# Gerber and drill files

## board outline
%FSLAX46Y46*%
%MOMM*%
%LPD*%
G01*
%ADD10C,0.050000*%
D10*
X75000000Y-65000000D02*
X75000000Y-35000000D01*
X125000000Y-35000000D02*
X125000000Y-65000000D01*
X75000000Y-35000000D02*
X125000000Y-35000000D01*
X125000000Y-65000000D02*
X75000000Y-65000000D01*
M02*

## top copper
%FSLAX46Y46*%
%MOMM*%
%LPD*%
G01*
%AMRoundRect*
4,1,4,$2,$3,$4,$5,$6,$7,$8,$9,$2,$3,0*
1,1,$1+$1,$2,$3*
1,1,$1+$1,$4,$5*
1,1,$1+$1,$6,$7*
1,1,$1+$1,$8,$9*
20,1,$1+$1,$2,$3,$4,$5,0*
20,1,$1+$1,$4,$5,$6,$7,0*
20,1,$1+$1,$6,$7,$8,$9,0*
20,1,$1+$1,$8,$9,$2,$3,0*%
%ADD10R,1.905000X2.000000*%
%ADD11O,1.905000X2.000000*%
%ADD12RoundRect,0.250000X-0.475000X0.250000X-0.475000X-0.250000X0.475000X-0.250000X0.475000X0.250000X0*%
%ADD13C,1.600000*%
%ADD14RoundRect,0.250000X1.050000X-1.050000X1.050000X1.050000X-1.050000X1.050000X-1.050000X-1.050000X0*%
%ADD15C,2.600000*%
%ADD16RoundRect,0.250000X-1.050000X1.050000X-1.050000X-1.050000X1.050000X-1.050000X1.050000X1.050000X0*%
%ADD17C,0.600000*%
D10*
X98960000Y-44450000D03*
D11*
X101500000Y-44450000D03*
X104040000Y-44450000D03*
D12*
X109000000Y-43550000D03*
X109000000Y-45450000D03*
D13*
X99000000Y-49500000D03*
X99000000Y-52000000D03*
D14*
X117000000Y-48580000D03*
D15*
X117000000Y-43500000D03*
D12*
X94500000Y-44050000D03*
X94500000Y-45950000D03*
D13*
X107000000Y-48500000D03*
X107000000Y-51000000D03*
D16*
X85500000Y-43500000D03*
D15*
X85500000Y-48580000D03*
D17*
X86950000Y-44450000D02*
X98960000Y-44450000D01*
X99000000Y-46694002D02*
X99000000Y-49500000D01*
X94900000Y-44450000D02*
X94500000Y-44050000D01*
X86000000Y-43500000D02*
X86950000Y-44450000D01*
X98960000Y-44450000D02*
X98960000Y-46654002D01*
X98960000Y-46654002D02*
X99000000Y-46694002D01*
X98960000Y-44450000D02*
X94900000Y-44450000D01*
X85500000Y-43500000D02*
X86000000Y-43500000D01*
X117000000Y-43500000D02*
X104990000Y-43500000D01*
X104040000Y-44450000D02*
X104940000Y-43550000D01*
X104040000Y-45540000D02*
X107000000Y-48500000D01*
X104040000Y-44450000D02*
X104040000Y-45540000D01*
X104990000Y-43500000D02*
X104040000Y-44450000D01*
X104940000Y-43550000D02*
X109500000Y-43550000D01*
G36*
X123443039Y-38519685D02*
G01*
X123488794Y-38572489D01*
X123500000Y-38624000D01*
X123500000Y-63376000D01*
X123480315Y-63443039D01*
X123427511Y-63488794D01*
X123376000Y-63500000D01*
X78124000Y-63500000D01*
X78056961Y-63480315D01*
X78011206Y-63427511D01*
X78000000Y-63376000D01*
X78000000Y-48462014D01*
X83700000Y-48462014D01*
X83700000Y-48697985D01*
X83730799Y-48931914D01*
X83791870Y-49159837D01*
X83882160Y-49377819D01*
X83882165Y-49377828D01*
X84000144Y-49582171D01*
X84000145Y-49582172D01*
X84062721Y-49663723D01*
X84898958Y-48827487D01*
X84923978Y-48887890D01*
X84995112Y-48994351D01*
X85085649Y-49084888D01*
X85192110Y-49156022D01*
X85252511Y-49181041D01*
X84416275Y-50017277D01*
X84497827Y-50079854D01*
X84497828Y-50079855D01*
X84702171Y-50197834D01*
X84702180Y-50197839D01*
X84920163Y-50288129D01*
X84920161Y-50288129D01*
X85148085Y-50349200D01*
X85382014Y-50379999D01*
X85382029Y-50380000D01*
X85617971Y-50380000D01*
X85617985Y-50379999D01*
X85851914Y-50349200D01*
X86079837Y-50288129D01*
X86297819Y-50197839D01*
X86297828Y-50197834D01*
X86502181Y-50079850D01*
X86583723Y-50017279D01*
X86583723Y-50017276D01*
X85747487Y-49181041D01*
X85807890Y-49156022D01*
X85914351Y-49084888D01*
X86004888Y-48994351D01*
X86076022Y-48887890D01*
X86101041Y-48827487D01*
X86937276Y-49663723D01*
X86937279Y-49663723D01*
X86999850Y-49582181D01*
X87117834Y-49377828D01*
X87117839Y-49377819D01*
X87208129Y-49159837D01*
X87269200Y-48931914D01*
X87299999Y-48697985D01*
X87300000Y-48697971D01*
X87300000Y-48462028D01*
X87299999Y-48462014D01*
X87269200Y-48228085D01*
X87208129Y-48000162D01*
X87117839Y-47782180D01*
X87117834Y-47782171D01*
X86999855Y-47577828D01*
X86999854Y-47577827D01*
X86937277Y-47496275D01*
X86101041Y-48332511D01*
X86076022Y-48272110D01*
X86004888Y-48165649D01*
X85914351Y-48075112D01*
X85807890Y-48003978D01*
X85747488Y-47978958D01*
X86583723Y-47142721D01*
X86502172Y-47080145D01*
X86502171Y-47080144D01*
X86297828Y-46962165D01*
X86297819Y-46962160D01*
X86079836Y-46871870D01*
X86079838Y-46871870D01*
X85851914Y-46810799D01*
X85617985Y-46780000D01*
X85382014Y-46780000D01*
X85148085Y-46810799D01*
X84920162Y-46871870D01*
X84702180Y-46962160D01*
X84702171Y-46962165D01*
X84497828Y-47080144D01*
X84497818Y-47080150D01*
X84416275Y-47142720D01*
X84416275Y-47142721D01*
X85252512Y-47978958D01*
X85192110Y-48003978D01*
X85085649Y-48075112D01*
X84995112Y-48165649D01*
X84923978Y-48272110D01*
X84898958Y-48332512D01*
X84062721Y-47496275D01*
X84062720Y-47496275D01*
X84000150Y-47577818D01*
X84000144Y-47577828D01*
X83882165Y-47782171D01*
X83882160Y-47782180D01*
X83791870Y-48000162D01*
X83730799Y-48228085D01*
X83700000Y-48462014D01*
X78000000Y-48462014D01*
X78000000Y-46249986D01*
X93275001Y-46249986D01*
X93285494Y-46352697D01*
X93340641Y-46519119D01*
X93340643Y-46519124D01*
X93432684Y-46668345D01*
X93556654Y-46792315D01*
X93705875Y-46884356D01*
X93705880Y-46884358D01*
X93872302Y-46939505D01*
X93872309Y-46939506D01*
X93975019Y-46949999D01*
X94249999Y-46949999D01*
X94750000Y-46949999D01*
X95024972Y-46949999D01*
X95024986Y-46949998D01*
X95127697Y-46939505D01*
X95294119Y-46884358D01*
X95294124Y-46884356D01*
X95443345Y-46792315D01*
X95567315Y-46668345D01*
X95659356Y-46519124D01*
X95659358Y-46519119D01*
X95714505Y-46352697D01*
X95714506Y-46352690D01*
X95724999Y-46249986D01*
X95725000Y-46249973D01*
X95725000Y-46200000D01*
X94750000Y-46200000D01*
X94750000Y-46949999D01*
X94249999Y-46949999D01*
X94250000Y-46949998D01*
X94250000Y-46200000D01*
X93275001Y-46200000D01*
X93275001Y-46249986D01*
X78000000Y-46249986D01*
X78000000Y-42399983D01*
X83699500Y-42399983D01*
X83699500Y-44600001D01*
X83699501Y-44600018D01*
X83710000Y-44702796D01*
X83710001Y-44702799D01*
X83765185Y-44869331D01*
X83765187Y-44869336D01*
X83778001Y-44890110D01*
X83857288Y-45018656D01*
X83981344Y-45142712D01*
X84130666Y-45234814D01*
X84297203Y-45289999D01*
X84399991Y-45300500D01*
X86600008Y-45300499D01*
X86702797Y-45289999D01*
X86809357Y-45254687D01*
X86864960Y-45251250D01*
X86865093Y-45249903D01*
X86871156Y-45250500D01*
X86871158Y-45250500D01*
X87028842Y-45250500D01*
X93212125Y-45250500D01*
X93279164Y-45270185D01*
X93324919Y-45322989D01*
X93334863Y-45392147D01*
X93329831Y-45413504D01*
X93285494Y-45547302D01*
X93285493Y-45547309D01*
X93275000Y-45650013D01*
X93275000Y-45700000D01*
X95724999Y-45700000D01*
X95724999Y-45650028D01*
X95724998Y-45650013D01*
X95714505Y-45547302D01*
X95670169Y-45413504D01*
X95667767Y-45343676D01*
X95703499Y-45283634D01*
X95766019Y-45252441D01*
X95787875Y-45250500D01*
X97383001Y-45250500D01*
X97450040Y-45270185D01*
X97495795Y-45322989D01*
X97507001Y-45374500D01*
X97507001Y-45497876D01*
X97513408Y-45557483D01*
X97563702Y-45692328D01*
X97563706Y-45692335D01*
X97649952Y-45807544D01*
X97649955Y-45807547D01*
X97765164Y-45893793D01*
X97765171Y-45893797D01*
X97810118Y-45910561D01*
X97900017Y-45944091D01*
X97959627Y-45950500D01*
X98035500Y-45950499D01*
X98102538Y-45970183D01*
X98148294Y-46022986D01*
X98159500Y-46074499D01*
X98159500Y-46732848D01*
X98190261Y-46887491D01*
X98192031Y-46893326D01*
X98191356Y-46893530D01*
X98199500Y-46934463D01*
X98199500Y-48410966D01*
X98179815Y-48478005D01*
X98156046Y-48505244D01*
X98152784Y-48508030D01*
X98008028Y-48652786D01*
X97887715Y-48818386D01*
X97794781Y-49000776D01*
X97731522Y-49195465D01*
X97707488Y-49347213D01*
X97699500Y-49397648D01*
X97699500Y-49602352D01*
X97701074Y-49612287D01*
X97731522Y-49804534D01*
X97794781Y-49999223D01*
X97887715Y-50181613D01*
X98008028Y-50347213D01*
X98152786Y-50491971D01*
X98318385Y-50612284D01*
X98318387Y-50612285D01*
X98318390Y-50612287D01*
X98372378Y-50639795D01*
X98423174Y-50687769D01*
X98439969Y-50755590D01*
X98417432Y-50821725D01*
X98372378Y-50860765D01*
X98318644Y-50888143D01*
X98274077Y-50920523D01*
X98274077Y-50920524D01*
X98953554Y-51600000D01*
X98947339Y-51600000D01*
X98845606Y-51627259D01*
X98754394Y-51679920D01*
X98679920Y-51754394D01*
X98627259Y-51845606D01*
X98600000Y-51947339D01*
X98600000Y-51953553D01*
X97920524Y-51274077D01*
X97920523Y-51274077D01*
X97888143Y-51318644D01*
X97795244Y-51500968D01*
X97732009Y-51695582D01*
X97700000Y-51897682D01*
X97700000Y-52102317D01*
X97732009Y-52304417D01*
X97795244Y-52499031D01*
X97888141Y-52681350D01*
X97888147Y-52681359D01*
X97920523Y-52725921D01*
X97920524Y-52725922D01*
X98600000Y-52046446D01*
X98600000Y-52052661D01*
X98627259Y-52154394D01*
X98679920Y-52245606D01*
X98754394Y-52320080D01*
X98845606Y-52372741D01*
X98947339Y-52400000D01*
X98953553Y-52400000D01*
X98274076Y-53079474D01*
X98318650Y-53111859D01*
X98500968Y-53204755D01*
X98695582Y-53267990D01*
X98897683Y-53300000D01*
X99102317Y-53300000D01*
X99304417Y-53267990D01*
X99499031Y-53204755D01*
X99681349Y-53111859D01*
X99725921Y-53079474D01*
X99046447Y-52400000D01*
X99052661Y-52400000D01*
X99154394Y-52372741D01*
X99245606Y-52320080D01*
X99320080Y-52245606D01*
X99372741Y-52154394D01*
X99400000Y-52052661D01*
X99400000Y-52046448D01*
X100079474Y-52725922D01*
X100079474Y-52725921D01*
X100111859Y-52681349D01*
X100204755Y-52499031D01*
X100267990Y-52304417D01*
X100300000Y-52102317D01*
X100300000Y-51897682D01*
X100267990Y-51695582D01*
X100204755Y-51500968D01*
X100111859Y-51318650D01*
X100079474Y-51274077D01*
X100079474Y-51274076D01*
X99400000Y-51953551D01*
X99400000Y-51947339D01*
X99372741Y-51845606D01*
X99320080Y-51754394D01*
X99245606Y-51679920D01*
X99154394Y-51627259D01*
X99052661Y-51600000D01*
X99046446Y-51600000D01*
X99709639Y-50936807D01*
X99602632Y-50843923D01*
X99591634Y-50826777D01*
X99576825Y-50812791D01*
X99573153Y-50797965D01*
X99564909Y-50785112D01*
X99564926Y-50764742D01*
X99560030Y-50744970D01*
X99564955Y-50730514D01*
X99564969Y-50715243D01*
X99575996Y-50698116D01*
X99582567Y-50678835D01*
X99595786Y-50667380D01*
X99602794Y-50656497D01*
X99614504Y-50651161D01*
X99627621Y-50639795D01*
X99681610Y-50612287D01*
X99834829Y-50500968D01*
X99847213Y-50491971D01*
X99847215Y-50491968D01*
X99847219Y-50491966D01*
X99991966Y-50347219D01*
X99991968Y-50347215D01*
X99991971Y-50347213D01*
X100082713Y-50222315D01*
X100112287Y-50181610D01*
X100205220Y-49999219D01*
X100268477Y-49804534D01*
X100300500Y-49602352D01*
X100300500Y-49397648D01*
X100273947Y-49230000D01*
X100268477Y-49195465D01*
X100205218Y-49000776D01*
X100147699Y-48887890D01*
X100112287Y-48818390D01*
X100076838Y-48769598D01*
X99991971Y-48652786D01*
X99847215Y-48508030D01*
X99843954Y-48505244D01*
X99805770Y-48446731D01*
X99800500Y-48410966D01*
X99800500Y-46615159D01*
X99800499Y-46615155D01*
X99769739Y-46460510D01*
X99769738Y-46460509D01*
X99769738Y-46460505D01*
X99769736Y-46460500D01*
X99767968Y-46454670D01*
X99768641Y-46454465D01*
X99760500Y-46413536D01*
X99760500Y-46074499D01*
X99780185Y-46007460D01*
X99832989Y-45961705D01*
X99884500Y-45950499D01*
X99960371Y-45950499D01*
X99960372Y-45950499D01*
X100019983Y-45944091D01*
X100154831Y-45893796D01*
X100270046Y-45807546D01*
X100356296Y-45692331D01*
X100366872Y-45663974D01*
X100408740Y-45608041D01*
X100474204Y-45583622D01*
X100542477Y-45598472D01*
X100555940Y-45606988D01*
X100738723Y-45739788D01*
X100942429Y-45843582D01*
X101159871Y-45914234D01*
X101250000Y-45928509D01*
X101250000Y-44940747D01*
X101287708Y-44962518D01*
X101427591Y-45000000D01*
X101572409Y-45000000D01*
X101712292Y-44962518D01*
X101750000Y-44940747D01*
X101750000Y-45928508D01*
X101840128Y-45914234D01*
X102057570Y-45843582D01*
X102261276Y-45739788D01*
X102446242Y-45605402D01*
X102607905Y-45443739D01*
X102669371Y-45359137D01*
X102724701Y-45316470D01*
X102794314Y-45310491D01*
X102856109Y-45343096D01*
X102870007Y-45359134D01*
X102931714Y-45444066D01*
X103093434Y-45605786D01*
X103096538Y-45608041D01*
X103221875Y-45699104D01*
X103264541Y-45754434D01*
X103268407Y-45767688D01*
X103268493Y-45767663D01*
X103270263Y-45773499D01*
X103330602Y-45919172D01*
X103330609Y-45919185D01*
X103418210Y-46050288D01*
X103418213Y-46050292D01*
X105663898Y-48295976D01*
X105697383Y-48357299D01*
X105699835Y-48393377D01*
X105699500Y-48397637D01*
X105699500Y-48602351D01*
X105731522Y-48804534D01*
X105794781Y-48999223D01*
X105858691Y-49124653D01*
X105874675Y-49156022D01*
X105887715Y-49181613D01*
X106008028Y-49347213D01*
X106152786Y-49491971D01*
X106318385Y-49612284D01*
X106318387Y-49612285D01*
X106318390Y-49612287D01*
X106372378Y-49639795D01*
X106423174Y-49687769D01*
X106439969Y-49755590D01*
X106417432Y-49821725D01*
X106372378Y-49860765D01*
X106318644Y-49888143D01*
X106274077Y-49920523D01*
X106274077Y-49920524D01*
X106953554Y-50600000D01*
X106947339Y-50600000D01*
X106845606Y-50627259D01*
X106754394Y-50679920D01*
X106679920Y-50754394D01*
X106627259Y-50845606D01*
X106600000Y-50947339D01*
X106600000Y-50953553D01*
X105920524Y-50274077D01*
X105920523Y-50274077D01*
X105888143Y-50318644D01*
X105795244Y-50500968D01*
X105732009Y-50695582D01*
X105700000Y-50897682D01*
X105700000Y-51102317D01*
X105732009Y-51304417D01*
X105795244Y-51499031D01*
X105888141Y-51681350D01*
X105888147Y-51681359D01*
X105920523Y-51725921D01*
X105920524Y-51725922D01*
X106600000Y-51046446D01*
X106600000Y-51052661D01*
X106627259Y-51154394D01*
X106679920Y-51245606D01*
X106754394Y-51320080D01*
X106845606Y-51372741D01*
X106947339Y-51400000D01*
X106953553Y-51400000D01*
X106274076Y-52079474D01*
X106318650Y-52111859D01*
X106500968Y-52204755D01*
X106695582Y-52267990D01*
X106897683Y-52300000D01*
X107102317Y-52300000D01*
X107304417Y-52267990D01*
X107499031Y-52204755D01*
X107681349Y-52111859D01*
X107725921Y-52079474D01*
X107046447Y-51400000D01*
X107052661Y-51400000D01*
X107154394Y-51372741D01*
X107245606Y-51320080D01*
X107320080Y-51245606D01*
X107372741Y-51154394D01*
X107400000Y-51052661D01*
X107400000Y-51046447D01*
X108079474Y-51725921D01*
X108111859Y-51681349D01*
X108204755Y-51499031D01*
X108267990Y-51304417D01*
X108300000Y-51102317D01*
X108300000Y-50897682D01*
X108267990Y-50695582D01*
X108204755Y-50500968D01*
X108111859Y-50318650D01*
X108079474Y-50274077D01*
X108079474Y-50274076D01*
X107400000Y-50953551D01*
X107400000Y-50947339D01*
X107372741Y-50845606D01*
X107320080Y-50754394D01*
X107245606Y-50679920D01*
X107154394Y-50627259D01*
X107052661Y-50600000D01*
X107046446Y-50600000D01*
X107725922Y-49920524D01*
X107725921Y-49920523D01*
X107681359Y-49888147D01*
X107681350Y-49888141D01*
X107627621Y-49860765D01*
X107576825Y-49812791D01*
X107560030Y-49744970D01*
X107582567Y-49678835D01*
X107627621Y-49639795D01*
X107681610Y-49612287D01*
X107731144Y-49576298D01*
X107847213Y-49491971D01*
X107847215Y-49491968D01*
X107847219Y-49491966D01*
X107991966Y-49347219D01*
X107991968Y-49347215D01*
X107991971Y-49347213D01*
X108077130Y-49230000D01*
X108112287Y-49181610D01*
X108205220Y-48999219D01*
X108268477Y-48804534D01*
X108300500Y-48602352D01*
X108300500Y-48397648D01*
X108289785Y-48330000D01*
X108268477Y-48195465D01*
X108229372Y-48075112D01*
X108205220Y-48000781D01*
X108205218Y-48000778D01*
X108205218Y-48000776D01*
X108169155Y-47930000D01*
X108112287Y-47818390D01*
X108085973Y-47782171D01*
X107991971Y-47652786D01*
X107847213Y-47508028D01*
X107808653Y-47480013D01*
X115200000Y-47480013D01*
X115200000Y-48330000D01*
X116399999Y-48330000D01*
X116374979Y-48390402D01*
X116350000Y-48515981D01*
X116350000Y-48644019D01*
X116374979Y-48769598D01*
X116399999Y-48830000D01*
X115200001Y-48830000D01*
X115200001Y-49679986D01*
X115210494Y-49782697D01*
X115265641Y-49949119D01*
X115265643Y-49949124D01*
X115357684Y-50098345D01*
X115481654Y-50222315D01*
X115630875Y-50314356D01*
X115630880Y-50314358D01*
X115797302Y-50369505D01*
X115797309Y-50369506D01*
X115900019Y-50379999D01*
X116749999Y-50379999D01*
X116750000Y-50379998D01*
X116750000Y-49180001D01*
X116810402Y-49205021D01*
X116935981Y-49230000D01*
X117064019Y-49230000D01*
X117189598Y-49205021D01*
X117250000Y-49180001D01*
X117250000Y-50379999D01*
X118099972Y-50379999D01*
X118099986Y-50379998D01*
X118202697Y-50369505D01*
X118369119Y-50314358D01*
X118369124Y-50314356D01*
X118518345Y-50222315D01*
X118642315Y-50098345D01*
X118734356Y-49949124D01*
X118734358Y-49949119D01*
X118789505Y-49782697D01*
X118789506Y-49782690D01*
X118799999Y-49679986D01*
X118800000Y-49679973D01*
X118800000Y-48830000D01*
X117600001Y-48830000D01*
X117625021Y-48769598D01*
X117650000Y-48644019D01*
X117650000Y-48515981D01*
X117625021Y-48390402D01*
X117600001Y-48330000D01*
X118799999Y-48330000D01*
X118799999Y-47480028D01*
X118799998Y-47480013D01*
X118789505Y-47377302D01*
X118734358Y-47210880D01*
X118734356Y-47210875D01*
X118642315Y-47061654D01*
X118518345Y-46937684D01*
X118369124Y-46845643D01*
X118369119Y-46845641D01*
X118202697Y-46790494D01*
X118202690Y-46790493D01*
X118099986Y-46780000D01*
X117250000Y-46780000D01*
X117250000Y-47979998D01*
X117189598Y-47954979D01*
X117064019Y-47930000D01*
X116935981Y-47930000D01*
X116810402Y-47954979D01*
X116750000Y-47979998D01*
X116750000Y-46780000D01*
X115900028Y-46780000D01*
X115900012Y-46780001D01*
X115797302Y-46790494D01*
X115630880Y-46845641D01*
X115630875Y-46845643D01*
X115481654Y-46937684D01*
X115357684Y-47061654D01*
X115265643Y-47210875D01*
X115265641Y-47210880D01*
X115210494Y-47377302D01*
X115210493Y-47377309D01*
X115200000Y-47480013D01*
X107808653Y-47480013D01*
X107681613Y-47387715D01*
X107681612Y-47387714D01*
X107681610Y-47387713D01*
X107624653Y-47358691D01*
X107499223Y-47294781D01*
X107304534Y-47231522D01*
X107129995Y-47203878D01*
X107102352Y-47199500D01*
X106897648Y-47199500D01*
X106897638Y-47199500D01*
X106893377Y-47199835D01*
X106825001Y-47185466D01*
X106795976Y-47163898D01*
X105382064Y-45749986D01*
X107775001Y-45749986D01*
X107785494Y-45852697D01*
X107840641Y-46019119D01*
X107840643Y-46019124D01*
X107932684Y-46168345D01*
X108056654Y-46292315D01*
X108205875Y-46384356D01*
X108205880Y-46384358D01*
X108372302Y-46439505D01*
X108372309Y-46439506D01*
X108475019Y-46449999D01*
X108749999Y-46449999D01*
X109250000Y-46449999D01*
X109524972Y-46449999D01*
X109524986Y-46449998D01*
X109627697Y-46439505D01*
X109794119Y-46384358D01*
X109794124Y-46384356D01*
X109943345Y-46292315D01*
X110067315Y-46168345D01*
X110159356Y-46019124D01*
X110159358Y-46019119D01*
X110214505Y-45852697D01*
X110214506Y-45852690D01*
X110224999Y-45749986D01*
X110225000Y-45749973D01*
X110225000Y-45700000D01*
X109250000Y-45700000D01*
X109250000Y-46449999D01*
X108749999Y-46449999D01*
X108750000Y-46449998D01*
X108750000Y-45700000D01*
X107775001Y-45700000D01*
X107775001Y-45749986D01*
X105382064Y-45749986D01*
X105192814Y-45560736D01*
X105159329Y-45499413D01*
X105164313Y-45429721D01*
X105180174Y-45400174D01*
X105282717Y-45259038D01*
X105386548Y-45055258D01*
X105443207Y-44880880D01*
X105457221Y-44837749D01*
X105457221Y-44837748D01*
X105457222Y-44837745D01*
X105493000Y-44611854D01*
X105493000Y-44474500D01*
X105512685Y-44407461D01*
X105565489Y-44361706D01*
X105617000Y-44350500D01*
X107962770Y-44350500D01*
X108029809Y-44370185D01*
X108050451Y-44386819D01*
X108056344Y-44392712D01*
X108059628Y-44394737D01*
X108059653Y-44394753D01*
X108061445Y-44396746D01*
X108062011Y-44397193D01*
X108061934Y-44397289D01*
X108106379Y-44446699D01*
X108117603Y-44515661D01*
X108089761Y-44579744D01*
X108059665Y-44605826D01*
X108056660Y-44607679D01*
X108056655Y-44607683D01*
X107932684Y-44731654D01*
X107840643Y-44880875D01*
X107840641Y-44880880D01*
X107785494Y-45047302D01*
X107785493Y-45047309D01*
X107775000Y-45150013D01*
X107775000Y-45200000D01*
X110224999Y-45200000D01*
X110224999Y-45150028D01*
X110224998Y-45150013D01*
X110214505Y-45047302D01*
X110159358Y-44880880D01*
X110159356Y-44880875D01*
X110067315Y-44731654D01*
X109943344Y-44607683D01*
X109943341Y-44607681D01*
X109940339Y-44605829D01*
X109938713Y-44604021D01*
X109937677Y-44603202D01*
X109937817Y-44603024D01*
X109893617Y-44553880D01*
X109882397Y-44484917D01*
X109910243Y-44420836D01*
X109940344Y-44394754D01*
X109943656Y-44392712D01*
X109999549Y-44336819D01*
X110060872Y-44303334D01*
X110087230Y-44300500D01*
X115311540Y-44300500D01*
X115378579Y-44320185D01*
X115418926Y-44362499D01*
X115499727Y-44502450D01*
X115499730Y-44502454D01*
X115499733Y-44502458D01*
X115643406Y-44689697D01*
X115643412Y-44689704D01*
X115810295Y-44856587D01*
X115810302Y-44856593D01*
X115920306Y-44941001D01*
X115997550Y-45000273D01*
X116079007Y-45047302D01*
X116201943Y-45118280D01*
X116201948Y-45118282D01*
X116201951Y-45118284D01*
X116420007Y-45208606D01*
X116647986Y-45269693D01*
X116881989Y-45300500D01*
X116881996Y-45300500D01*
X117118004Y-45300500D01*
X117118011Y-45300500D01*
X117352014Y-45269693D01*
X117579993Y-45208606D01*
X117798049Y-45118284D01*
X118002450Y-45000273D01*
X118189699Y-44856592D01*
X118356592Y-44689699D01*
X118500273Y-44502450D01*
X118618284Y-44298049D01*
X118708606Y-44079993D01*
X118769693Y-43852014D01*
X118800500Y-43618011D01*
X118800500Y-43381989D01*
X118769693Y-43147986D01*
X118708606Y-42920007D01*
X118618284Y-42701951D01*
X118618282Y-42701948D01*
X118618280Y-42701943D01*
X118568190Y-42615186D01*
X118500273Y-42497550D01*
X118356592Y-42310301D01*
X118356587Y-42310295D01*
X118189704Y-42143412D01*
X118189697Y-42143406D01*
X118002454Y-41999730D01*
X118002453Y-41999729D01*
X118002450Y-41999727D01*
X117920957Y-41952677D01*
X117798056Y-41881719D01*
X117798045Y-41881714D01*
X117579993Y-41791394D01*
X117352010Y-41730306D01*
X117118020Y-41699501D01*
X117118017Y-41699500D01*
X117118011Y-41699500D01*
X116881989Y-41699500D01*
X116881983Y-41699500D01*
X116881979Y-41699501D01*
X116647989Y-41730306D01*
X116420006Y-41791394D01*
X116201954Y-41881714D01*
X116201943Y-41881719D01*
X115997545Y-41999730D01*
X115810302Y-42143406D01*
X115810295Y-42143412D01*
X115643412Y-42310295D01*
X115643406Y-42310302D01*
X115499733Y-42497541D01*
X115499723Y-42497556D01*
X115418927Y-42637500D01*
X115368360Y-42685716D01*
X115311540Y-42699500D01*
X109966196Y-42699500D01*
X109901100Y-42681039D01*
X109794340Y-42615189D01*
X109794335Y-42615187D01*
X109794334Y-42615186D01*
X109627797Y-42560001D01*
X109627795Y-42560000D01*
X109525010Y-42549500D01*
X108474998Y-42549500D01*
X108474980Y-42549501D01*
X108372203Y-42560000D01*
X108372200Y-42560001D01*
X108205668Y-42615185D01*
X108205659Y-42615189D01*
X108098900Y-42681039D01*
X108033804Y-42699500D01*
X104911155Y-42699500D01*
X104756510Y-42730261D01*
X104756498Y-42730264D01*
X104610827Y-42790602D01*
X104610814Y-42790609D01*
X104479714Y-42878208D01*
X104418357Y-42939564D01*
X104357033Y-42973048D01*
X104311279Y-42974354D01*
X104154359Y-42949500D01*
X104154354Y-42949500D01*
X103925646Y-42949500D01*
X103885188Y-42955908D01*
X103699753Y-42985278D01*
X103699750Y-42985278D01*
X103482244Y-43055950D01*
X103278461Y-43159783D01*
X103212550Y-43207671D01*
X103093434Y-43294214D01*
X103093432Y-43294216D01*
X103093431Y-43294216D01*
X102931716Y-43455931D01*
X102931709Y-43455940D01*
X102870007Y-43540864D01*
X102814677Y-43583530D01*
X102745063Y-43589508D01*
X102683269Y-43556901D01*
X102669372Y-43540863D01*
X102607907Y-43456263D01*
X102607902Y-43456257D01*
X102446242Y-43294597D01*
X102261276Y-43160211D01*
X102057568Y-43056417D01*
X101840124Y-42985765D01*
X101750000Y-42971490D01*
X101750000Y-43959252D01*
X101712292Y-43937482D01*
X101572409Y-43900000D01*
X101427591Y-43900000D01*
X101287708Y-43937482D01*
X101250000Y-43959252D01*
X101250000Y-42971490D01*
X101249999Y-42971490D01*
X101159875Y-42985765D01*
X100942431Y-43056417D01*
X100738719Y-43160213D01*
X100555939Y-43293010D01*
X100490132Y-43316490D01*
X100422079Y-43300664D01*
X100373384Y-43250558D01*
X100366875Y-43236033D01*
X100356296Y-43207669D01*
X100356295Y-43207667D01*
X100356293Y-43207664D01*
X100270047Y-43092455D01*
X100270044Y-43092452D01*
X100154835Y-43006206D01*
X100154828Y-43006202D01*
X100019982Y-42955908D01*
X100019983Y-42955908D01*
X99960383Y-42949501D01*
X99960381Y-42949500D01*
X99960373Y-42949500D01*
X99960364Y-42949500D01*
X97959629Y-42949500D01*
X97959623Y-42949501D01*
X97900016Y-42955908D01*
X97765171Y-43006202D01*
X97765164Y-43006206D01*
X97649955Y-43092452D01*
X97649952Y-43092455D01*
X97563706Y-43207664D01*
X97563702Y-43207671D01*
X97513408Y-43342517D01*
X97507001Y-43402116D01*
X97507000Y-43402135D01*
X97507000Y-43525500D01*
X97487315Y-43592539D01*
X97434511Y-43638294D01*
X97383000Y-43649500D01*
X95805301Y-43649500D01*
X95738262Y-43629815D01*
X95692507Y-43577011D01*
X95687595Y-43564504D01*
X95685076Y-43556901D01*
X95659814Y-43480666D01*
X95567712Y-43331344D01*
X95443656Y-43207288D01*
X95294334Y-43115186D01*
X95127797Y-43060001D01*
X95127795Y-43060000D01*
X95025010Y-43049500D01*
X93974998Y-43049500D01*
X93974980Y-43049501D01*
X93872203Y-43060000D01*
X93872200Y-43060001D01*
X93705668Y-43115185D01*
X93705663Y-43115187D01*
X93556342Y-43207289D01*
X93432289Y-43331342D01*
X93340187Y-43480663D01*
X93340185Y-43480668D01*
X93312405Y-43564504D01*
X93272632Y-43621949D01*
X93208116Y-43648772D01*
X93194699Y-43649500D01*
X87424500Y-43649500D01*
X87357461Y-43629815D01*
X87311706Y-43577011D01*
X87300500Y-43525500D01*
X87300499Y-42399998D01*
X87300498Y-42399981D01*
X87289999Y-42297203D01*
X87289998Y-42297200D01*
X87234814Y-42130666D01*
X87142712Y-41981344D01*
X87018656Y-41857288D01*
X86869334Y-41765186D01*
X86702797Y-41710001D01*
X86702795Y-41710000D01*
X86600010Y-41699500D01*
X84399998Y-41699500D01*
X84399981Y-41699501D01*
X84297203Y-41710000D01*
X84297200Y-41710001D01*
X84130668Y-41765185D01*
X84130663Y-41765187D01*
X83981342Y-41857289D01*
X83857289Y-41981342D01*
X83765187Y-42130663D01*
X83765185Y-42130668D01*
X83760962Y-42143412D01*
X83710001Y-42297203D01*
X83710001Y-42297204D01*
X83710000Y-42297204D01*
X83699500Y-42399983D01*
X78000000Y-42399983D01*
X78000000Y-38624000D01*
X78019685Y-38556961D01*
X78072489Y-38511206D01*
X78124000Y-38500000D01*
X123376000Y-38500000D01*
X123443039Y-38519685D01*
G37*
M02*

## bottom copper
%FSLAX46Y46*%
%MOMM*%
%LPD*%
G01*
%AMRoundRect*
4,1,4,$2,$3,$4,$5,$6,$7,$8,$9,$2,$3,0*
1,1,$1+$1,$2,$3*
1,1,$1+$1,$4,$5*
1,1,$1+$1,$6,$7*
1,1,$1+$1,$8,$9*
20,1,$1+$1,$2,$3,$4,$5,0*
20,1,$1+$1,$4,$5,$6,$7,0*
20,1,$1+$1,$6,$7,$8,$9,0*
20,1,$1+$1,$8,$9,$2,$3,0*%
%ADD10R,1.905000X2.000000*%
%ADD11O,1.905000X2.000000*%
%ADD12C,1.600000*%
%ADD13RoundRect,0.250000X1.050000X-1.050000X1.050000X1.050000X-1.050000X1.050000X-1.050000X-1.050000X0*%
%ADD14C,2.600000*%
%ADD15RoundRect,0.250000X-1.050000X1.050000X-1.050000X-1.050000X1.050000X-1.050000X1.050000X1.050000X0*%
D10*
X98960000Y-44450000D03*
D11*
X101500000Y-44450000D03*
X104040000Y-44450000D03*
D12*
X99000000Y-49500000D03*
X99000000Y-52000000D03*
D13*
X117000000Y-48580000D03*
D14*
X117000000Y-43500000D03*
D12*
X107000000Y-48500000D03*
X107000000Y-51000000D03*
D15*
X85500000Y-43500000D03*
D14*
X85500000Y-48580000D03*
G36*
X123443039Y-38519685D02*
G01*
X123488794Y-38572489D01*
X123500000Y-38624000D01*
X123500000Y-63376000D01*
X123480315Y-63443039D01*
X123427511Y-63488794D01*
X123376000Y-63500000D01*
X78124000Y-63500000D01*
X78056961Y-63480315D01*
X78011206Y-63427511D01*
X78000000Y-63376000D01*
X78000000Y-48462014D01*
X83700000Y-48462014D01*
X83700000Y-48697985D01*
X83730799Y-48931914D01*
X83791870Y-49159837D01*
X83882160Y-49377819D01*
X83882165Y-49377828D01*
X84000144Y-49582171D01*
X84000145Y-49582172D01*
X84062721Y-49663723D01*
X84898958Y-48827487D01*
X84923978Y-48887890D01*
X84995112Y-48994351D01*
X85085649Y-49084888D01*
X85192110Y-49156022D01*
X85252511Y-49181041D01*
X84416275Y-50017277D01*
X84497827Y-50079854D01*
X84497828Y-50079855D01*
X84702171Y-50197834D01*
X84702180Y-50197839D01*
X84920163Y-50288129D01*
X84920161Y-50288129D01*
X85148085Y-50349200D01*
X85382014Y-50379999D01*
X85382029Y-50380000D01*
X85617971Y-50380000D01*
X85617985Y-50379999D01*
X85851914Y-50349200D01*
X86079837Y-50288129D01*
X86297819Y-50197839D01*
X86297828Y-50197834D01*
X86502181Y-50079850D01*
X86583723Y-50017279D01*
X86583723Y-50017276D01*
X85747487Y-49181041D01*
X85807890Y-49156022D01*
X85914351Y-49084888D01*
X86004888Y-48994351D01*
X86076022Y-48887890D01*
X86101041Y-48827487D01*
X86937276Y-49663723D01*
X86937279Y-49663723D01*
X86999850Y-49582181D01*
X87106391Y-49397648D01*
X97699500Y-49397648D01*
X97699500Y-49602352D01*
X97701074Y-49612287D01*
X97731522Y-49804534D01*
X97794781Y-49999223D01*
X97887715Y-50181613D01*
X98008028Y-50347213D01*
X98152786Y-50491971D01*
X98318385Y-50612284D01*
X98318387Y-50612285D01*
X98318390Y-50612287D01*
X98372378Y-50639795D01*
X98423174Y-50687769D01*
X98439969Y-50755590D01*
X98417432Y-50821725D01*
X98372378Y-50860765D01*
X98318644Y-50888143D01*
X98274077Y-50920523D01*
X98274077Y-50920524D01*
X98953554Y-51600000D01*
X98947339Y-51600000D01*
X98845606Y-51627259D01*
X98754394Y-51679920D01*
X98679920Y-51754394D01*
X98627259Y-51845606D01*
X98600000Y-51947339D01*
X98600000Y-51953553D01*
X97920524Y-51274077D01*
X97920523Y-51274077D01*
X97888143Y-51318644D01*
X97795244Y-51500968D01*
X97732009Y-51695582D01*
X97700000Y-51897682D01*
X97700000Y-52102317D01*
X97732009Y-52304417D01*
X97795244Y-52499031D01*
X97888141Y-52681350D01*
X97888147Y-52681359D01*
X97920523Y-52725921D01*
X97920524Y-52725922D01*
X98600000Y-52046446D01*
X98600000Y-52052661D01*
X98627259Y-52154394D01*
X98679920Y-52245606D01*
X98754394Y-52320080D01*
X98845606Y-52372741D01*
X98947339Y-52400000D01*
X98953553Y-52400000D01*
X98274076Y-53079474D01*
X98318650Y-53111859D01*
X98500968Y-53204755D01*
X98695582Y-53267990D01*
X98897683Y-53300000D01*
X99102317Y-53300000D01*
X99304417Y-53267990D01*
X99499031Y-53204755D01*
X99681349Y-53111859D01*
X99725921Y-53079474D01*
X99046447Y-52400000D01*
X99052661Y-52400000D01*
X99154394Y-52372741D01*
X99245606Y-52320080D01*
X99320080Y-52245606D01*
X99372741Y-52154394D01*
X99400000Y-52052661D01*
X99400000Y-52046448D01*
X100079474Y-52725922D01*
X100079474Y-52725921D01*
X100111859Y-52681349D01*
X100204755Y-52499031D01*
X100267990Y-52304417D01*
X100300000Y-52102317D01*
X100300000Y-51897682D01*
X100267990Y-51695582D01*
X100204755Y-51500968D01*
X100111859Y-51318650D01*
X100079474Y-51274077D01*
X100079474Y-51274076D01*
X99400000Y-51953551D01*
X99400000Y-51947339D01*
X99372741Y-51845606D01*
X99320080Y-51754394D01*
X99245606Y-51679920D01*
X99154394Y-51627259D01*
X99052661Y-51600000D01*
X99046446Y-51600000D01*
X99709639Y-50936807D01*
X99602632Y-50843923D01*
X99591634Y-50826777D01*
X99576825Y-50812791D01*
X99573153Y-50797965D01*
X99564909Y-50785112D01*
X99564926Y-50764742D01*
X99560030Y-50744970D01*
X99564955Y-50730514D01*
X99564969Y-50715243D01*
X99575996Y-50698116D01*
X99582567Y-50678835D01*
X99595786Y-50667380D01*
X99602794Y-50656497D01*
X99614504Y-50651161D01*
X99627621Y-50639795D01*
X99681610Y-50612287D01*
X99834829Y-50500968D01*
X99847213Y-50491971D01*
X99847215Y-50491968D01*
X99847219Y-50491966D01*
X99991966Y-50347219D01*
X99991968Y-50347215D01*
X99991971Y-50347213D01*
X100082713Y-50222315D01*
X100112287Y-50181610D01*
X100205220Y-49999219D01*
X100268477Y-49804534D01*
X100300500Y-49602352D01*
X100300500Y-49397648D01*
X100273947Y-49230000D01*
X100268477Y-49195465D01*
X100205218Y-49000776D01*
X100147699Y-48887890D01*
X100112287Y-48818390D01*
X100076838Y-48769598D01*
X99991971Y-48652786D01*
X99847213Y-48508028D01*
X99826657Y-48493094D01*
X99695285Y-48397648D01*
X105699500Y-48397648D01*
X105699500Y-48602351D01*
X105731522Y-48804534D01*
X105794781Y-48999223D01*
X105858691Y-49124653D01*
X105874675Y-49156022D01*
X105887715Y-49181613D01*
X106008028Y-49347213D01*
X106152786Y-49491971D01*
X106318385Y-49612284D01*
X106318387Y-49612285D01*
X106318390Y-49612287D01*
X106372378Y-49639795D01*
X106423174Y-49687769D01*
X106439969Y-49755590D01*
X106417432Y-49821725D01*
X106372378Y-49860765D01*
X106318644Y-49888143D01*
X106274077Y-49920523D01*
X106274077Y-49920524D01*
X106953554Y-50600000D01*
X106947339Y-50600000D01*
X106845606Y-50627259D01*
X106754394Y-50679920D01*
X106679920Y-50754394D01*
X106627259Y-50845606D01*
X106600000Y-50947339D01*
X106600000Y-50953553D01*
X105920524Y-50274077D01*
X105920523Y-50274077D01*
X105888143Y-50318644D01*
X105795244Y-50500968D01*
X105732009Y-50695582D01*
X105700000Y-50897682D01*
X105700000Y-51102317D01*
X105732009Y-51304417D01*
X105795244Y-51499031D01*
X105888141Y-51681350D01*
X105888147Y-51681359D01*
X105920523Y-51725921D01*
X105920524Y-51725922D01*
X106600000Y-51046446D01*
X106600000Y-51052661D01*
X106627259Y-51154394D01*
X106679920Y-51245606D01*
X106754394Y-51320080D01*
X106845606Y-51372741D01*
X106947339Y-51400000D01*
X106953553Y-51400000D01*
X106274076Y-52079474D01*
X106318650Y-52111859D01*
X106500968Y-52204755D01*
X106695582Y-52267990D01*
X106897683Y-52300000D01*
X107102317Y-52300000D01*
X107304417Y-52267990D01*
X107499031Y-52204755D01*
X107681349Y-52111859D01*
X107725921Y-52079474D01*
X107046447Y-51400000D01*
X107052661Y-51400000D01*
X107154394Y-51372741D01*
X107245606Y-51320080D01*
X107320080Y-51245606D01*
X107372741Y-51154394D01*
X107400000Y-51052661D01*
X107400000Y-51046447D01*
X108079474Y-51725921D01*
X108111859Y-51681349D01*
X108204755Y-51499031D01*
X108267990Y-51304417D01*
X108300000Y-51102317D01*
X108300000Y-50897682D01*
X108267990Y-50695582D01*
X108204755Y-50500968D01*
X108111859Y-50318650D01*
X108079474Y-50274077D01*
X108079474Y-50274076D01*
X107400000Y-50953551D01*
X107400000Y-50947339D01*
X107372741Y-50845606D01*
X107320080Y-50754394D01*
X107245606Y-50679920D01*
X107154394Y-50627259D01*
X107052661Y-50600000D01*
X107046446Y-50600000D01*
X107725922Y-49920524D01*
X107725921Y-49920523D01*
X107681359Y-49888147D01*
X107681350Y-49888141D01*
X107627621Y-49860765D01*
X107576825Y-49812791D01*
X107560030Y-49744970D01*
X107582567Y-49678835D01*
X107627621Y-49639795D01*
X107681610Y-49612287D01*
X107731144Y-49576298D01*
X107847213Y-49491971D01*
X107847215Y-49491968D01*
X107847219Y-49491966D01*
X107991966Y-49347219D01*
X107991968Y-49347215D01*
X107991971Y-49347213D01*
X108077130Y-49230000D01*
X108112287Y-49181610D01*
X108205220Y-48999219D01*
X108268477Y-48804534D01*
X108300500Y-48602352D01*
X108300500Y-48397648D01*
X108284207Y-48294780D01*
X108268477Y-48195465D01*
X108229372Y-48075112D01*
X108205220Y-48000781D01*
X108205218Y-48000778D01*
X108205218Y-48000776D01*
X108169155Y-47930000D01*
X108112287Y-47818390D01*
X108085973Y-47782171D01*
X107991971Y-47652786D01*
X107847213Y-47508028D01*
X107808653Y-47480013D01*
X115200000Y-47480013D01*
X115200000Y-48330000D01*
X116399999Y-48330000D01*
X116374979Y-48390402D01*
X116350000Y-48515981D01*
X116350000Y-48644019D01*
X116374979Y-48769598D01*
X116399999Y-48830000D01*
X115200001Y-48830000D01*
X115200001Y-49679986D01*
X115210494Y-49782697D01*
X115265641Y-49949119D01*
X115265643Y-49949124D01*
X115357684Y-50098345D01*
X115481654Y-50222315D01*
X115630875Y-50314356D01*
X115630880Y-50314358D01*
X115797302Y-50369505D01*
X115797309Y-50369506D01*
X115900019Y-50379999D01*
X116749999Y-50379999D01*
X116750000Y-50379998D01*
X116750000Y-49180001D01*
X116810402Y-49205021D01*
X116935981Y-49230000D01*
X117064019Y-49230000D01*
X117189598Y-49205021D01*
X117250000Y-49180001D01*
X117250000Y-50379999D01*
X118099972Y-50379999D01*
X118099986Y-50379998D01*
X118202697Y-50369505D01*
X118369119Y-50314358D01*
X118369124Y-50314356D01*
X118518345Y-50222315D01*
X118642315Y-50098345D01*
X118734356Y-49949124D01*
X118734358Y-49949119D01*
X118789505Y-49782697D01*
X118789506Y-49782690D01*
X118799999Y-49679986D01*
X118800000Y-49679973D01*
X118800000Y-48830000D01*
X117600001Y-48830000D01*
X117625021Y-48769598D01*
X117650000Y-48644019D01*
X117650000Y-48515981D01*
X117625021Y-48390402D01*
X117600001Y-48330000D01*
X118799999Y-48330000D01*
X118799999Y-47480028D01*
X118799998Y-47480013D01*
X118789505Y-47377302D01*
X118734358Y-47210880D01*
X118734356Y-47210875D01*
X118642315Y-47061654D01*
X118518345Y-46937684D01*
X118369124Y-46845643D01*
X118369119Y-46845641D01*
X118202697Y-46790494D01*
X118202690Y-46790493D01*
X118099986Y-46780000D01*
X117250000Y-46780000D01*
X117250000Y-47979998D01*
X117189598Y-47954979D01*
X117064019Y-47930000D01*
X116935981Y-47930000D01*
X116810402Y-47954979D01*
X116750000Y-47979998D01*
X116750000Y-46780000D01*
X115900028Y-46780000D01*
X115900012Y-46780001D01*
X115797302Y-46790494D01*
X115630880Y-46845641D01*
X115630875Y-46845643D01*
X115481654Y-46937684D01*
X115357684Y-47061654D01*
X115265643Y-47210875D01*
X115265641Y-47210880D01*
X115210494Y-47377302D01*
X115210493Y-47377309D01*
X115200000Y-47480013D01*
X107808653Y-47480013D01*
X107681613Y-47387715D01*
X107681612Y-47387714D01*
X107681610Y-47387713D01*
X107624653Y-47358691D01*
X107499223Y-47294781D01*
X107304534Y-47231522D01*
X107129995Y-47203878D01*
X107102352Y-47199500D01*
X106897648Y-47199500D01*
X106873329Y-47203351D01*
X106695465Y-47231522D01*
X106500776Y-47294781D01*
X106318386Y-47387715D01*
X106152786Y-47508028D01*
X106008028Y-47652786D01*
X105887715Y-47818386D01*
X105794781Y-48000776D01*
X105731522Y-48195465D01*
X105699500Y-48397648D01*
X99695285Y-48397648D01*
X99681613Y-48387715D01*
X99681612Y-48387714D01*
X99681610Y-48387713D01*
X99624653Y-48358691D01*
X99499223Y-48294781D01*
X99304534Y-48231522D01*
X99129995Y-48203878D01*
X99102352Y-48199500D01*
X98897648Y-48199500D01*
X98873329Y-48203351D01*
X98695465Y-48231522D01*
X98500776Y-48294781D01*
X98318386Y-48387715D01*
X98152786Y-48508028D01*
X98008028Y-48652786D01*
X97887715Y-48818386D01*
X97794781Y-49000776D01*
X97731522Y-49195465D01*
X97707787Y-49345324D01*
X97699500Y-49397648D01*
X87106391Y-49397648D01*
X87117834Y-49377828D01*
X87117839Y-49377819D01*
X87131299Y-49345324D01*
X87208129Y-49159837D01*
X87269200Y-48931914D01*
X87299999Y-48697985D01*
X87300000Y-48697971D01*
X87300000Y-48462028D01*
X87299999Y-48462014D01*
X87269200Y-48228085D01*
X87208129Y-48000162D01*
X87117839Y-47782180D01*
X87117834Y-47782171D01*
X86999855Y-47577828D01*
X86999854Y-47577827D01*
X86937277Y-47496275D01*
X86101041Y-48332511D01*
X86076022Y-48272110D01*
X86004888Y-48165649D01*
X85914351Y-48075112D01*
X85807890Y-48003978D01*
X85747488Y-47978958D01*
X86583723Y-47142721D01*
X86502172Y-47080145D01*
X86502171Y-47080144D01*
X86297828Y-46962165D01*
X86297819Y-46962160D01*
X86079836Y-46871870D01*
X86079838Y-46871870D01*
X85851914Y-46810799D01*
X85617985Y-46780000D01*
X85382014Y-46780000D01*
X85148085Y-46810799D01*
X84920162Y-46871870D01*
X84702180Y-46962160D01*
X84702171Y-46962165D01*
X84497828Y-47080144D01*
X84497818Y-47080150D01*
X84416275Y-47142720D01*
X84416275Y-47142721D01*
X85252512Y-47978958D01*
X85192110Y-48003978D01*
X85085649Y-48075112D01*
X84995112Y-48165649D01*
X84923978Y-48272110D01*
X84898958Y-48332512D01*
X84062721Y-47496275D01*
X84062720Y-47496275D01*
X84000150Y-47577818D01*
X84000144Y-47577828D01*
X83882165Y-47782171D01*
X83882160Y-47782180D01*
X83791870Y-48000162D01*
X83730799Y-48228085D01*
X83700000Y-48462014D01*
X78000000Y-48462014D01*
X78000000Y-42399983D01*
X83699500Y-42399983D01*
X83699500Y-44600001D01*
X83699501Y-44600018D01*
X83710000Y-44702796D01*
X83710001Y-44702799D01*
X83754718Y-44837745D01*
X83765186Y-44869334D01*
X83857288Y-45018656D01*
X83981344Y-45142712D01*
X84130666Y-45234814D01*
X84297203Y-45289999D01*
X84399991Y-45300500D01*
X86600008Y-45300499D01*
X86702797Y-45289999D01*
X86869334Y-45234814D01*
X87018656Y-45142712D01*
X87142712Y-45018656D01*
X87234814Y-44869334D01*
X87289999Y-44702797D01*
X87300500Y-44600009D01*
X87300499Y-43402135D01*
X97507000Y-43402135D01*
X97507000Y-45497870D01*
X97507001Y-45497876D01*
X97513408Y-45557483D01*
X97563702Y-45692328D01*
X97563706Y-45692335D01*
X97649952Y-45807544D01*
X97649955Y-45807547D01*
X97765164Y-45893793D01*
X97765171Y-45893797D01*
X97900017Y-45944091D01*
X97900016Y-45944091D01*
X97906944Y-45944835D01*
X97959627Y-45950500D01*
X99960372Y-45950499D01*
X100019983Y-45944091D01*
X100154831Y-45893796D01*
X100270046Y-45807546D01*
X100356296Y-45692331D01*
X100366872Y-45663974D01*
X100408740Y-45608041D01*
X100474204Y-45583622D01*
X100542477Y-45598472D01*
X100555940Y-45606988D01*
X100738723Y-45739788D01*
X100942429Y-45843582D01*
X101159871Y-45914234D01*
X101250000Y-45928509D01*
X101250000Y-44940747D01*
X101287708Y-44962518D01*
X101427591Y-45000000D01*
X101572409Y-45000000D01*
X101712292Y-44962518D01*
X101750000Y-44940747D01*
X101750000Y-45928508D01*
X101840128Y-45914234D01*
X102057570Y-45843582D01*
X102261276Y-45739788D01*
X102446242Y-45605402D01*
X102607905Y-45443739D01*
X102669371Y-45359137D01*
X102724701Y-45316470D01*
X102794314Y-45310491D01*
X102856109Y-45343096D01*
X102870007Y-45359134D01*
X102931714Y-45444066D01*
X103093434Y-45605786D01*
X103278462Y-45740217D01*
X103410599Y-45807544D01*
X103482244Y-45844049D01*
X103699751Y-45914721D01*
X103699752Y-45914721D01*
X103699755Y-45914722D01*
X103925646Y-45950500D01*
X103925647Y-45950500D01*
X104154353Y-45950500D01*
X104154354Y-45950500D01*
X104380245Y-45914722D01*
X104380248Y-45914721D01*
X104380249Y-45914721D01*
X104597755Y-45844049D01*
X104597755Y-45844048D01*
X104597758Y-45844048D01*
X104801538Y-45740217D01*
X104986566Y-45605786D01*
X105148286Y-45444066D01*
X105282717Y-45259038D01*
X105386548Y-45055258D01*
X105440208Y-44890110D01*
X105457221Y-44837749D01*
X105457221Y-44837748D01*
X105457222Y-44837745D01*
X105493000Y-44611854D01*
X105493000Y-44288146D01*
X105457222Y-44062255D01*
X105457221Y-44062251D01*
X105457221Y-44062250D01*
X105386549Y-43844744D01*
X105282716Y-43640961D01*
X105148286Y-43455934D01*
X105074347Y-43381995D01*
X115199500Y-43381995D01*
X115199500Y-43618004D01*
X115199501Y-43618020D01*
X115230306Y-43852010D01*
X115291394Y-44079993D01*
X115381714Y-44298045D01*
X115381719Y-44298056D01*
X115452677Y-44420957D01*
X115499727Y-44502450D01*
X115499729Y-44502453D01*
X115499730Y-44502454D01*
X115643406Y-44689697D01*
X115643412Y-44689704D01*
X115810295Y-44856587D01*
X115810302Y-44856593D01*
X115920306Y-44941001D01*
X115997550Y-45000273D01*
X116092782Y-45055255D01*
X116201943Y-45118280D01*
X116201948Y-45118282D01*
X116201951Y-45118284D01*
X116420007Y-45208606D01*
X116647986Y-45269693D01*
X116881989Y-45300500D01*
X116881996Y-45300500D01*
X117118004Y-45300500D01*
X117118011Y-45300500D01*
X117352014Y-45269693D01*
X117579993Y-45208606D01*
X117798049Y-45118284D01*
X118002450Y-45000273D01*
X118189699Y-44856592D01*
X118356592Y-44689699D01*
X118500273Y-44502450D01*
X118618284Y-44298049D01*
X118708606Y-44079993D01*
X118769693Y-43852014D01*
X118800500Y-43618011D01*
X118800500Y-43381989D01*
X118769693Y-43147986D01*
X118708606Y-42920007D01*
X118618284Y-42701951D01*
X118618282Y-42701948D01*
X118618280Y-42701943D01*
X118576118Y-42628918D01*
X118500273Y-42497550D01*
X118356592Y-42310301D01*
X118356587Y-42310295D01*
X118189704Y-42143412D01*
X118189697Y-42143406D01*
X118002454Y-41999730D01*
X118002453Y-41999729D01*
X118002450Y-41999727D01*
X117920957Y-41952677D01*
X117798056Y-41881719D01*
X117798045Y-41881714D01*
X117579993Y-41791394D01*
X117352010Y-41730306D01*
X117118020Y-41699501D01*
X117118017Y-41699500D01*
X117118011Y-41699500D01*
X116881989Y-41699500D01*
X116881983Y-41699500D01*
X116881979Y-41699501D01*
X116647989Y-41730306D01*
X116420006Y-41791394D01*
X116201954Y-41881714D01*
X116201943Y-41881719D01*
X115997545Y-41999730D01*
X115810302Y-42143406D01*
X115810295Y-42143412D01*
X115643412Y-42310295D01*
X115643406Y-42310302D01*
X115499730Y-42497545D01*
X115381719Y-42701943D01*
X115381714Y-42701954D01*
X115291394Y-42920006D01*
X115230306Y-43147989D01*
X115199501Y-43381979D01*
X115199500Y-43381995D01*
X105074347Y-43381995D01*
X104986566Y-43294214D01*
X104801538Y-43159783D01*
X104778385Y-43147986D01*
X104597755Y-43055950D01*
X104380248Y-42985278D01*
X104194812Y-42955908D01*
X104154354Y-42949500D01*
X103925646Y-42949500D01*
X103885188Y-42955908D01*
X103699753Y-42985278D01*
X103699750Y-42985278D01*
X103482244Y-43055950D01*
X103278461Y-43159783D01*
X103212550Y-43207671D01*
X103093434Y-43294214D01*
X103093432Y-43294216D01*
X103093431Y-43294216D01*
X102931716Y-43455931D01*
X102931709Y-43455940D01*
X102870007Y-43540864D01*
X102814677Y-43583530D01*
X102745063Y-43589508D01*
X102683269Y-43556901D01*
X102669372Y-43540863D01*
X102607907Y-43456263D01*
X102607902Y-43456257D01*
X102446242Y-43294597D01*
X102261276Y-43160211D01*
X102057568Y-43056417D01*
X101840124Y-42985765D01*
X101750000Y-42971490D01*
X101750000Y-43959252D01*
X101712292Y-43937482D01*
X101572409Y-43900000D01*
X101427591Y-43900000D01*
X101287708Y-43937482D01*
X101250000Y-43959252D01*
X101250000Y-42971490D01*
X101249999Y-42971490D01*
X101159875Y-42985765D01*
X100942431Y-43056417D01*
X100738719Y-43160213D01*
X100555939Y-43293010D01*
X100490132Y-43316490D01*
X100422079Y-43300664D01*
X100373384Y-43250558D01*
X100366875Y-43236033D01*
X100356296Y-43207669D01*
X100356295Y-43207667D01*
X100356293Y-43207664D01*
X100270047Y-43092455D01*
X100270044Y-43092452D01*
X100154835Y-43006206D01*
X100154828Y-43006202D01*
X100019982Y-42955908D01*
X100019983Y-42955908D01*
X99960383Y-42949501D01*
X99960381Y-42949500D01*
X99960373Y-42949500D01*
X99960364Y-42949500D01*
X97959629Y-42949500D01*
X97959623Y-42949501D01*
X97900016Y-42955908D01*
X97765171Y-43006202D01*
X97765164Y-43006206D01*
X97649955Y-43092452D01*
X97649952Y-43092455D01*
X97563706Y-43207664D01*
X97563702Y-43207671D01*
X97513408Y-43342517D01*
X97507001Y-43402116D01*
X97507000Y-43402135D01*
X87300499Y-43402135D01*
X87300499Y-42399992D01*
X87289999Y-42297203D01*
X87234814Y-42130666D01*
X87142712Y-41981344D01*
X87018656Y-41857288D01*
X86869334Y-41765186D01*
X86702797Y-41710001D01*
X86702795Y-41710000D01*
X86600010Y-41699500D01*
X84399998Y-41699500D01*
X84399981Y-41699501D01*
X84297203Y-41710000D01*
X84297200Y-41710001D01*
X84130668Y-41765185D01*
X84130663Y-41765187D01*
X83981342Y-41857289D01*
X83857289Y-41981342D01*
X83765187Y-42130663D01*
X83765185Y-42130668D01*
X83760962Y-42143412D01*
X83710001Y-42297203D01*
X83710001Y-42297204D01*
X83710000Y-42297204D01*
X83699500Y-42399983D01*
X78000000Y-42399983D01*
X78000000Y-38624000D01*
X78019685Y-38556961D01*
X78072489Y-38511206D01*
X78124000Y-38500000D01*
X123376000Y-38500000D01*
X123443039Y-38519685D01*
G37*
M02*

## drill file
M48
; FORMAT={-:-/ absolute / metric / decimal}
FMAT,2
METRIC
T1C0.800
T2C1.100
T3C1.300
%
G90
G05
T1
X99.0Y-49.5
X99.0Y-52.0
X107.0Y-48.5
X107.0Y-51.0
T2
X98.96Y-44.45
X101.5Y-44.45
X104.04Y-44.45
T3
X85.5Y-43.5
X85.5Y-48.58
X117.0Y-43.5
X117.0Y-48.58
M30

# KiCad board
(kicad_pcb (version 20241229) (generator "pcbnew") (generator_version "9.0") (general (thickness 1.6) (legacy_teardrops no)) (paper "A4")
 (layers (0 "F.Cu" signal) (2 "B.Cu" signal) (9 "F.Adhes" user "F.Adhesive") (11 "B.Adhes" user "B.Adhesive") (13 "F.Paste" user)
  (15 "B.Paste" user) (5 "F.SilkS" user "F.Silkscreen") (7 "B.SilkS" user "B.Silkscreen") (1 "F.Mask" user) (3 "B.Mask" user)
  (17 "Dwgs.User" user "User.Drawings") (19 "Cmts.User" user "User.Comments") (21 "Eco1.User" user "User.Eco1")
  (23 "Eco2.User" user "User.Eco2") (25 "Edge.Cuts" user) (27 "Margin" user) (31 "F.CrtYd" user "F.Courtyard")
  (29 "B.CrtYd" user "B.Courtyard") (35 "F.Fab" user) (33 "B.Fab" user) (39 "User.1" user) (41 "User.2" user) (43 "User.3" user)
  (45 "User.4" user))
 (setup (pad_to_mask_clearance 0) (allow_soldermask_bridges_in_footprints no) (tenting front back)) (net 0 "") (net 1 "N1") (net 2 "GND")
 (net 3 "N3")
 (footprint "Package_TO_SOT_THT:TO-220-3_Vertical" (layer "F.Cu") (at 98.96 44.45)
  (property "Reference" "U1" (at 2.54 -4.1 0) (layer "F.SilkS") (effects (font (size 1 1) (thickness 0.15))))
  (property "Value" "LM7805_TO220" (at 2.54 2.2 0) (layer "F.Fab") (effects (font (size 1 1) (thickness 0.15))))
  (pad "1" thru_hole rect (at 0 0) (size 1.905 2) (drill 1.1) (layers "*.Cu" "*.Mask") (remove_unused_layers no) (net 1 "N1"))
  (pad "2" thru_hole oval (at 2.54 0) (size 1.905 2) (drill 1.1) (layers "*.Cu" "*.Mask") (remove_unused_layers no) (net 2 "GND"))
  (pad "3" thru_hole oval (at 5.08 0) (size 1.905 2) (drill 1.1) (layers "*.Cu" "*.Mask") (remove_unused_layers no) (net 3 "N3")))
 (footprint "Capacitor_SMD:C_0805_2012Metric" (layer "F.Cu") (at 109 44.5 -90)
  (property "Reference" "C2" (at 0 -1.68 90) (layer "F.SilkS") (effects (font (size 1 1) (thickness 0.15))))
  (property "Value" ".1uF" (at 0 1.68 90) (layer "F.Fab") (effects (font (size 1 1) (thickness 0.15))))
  (pad "1" smd roundrect (at -0.95 0 270) (size 1 1.45) (layers "F.Cu" "F.Mask" "F.Paste") (roundrect_rratio 0.25) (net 3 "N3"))
  (pad "2" smd roundrect (at 0.95 0 270) (size 1 1.45) (layers "F.Cu" "F.Mask" "F.Paste") (roundrect_rratio 0.25) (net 2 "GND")))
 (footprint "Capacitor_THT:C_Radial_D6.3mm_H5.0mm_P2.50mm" (layer "F.Cu") (at 99 49.5 -90)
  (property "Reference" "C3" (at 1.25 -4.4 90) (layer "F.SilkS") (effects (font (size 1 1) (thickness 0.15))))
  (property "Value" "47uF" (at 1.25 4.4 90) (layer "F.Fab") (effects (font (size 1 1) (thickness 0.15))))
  (pad "1" thru_hole circle (at 0 0 270) (size 1.6 1.6) (drill 0.8) (layers "*.Cu" "*.Mask") (remove_unused_layers no) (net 1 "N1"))
  (pad "2" thru_hole circle (at 2.5 0 270) (size 1.6 1.6) (drill 0.8) (layers "*.Cu" "*.Mask") (remove_unused_layers no) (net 2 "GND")))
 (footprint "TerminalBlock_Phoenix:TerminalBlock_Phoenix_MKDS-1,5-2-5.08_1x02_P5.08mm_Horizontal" (layer "F.Cu") (at 117 48.58 90)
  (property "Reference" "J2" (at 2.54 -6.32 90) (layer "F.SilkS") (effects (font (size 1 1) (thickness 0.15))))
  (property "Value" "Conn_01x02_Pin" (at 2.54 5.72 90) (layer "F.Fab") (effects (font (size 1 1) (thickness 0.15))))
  (pad "1" thru_hole roundrect (at 0 0 90) (size 2.6 2.6) (drill 1.3) (layers "*.Cu" "*.Mask") (remove_unused_layers no)
   (roundrect_rratio 0.096154) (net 2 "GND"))
  (pad "2" thru_hole circle (at 5.08 0 90) (size 2.6 2.6) (drill 1.3) (layers "*.Cu" "*.Mask") (remove_unused_layers no) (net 3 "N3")))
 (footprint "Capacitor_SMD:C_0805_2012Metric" (layer "F.Cu") (at 94.5 45 -90)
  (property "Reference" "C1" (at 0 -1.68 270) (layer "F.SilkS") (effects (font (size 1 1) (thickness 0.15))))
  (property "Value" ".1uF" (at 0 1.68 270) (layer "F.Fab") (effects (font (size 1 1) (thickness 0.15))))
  (pad "1" smd roundrect (at -0.95 0 270) (size 1 1.45) (layers "F.Cu" "F.Mask" "F.Paste") (roundrect_rratio 0.25) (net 1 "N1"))
  (pad "2" smd roundrect (at 0.95 0 270) (size 1 1.45) (layers "F.Cu" "F.Mask" "F.Paste") (roundrect_rratio 0.25) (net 2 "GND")))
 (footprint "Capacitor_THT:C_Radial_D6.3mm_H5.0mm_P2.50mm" (layer "F.Cu") (at 107 48.5 -90)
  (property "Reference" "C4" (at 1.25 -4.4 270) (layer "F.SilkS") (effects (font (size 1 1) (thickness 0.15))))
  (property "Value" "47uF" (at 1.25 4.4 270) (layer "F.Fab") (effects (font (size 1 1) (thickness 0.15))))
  (pad "1" thru_hole circle (at 0 0 270) (size 1.6 1.6) (drill 0.8) (layers "*.Cu" "*.Mask") (remove_unused_layers no) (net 3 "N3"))
  (pad "2" thru_hole circle (at 2.5 0 270) (size 1.6 1.6) (drill 0.8) (layers "*.Cu" "*.Mask") (remove_unused_layers no) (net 2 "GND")))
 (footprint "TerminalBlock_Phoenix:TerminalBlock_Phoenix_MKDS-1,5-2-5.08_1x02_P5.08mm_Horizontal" (layer "F.Cu") (at 85.5 43.5 -90)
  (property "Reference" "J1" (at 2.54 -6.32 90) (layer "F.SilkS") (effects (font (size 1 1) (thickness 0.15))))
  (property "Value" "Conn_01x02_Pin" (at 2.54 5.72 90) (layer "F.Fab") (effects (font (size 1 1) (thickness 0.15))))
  (pad "1" thru_hole roundrect (at 0 0 270) (size 2.6 2.6) (drill 1.3) (layers "*.Cu" "*.Mask") (remove_unused_layers no)
   (roundrect_rratio 0.096154) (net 1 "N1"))
  (pad "2" thru_hole circle (at 5.08 0 270) (size 2.6 2.6) (drill 1.3) (layers "*.Cu" "*.Mask") (remove_unused_layers no) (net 2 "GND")))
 (gr_line (start 75 65) (end 75 35) (stroke (width 0.05) (type default)) (layer "Edge.Cuts"))
 (gr_line (start 125 35) (end 125 65) (stroke (width 0.05) (type default)) (layer "Edge.Cuts"))
 (gr_line (start 75 35) (end 125 35) (stroke (width 0.05) (type default)) (layer "Edge.Cuts"))
 (gr_line (start 125 65) (end 75 65) (stroke (width 0.05) (type default)) (layer "Edge.Cuts"))
 (segment (start 86.95 44.45) (end 98.96 44.45) (width 0.6) (layer "F.Cu") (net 1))
 (segment (start 99 46.694002) (end 99 49.5) (width 0.6) (layer "F.Cu") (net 1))
 (segment (start 94.9 44.45) (end 94.5 44.05) (width 0.6) (layer "F.Cu") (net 1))
 (segment (start 86 43.5) (end 86.95 44.45) (width 0.6) (layer "F.Cu") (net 1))
 (segment (start 98.96 44.45) (end 98.96 46.654002) (width 0.6) (layer "F.Cu") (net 1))
 (segment (start 98.96 46.654002) (end 99 46.694002) (width 0.6) (layer "F.Cu") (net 1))
 (segment (start 98.96 44.45) (end 94.9 44.45) (width 0.6) (layer "F.Cu") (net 1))
 (segment (start 85.5 43.5) (end 86 43.5) (width 0.6) (layer "F.Cu") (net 1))
 (segment (start 117 43.5) (end 104.99 43.5) (width 0.6) (layer "F.Cu") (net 3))
 (segment (start 104.04 44.45) (end 104.94 43.55) (width 0.6) (layer "F.Cu") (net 3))
 (segment (start 104.04 45.54) (end 107 48.5) (width 0.6) (layer "F.Cu") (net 3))
 (segment (start 104.04 44.45) (end 104.04 45.54) (width 0.6) (layer "F.Cu") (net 3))
 (segment (start 104.99 43.5) (end 104.04 44.45) (width 0.6) (layer "F.Cu") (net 3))
 (segment (start 104.94 43.55) (end 109.5 43.55) (width 0.6) (layer "F.Cu") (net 3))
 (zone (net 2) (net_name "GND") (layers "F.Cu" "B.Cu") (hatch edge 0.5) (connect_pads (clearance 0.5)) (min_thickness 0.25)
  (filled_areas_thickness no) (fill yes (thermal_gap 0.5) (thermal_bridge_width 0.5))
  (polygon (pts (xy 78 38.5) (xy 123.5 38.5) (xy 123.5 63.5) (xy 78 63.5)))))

